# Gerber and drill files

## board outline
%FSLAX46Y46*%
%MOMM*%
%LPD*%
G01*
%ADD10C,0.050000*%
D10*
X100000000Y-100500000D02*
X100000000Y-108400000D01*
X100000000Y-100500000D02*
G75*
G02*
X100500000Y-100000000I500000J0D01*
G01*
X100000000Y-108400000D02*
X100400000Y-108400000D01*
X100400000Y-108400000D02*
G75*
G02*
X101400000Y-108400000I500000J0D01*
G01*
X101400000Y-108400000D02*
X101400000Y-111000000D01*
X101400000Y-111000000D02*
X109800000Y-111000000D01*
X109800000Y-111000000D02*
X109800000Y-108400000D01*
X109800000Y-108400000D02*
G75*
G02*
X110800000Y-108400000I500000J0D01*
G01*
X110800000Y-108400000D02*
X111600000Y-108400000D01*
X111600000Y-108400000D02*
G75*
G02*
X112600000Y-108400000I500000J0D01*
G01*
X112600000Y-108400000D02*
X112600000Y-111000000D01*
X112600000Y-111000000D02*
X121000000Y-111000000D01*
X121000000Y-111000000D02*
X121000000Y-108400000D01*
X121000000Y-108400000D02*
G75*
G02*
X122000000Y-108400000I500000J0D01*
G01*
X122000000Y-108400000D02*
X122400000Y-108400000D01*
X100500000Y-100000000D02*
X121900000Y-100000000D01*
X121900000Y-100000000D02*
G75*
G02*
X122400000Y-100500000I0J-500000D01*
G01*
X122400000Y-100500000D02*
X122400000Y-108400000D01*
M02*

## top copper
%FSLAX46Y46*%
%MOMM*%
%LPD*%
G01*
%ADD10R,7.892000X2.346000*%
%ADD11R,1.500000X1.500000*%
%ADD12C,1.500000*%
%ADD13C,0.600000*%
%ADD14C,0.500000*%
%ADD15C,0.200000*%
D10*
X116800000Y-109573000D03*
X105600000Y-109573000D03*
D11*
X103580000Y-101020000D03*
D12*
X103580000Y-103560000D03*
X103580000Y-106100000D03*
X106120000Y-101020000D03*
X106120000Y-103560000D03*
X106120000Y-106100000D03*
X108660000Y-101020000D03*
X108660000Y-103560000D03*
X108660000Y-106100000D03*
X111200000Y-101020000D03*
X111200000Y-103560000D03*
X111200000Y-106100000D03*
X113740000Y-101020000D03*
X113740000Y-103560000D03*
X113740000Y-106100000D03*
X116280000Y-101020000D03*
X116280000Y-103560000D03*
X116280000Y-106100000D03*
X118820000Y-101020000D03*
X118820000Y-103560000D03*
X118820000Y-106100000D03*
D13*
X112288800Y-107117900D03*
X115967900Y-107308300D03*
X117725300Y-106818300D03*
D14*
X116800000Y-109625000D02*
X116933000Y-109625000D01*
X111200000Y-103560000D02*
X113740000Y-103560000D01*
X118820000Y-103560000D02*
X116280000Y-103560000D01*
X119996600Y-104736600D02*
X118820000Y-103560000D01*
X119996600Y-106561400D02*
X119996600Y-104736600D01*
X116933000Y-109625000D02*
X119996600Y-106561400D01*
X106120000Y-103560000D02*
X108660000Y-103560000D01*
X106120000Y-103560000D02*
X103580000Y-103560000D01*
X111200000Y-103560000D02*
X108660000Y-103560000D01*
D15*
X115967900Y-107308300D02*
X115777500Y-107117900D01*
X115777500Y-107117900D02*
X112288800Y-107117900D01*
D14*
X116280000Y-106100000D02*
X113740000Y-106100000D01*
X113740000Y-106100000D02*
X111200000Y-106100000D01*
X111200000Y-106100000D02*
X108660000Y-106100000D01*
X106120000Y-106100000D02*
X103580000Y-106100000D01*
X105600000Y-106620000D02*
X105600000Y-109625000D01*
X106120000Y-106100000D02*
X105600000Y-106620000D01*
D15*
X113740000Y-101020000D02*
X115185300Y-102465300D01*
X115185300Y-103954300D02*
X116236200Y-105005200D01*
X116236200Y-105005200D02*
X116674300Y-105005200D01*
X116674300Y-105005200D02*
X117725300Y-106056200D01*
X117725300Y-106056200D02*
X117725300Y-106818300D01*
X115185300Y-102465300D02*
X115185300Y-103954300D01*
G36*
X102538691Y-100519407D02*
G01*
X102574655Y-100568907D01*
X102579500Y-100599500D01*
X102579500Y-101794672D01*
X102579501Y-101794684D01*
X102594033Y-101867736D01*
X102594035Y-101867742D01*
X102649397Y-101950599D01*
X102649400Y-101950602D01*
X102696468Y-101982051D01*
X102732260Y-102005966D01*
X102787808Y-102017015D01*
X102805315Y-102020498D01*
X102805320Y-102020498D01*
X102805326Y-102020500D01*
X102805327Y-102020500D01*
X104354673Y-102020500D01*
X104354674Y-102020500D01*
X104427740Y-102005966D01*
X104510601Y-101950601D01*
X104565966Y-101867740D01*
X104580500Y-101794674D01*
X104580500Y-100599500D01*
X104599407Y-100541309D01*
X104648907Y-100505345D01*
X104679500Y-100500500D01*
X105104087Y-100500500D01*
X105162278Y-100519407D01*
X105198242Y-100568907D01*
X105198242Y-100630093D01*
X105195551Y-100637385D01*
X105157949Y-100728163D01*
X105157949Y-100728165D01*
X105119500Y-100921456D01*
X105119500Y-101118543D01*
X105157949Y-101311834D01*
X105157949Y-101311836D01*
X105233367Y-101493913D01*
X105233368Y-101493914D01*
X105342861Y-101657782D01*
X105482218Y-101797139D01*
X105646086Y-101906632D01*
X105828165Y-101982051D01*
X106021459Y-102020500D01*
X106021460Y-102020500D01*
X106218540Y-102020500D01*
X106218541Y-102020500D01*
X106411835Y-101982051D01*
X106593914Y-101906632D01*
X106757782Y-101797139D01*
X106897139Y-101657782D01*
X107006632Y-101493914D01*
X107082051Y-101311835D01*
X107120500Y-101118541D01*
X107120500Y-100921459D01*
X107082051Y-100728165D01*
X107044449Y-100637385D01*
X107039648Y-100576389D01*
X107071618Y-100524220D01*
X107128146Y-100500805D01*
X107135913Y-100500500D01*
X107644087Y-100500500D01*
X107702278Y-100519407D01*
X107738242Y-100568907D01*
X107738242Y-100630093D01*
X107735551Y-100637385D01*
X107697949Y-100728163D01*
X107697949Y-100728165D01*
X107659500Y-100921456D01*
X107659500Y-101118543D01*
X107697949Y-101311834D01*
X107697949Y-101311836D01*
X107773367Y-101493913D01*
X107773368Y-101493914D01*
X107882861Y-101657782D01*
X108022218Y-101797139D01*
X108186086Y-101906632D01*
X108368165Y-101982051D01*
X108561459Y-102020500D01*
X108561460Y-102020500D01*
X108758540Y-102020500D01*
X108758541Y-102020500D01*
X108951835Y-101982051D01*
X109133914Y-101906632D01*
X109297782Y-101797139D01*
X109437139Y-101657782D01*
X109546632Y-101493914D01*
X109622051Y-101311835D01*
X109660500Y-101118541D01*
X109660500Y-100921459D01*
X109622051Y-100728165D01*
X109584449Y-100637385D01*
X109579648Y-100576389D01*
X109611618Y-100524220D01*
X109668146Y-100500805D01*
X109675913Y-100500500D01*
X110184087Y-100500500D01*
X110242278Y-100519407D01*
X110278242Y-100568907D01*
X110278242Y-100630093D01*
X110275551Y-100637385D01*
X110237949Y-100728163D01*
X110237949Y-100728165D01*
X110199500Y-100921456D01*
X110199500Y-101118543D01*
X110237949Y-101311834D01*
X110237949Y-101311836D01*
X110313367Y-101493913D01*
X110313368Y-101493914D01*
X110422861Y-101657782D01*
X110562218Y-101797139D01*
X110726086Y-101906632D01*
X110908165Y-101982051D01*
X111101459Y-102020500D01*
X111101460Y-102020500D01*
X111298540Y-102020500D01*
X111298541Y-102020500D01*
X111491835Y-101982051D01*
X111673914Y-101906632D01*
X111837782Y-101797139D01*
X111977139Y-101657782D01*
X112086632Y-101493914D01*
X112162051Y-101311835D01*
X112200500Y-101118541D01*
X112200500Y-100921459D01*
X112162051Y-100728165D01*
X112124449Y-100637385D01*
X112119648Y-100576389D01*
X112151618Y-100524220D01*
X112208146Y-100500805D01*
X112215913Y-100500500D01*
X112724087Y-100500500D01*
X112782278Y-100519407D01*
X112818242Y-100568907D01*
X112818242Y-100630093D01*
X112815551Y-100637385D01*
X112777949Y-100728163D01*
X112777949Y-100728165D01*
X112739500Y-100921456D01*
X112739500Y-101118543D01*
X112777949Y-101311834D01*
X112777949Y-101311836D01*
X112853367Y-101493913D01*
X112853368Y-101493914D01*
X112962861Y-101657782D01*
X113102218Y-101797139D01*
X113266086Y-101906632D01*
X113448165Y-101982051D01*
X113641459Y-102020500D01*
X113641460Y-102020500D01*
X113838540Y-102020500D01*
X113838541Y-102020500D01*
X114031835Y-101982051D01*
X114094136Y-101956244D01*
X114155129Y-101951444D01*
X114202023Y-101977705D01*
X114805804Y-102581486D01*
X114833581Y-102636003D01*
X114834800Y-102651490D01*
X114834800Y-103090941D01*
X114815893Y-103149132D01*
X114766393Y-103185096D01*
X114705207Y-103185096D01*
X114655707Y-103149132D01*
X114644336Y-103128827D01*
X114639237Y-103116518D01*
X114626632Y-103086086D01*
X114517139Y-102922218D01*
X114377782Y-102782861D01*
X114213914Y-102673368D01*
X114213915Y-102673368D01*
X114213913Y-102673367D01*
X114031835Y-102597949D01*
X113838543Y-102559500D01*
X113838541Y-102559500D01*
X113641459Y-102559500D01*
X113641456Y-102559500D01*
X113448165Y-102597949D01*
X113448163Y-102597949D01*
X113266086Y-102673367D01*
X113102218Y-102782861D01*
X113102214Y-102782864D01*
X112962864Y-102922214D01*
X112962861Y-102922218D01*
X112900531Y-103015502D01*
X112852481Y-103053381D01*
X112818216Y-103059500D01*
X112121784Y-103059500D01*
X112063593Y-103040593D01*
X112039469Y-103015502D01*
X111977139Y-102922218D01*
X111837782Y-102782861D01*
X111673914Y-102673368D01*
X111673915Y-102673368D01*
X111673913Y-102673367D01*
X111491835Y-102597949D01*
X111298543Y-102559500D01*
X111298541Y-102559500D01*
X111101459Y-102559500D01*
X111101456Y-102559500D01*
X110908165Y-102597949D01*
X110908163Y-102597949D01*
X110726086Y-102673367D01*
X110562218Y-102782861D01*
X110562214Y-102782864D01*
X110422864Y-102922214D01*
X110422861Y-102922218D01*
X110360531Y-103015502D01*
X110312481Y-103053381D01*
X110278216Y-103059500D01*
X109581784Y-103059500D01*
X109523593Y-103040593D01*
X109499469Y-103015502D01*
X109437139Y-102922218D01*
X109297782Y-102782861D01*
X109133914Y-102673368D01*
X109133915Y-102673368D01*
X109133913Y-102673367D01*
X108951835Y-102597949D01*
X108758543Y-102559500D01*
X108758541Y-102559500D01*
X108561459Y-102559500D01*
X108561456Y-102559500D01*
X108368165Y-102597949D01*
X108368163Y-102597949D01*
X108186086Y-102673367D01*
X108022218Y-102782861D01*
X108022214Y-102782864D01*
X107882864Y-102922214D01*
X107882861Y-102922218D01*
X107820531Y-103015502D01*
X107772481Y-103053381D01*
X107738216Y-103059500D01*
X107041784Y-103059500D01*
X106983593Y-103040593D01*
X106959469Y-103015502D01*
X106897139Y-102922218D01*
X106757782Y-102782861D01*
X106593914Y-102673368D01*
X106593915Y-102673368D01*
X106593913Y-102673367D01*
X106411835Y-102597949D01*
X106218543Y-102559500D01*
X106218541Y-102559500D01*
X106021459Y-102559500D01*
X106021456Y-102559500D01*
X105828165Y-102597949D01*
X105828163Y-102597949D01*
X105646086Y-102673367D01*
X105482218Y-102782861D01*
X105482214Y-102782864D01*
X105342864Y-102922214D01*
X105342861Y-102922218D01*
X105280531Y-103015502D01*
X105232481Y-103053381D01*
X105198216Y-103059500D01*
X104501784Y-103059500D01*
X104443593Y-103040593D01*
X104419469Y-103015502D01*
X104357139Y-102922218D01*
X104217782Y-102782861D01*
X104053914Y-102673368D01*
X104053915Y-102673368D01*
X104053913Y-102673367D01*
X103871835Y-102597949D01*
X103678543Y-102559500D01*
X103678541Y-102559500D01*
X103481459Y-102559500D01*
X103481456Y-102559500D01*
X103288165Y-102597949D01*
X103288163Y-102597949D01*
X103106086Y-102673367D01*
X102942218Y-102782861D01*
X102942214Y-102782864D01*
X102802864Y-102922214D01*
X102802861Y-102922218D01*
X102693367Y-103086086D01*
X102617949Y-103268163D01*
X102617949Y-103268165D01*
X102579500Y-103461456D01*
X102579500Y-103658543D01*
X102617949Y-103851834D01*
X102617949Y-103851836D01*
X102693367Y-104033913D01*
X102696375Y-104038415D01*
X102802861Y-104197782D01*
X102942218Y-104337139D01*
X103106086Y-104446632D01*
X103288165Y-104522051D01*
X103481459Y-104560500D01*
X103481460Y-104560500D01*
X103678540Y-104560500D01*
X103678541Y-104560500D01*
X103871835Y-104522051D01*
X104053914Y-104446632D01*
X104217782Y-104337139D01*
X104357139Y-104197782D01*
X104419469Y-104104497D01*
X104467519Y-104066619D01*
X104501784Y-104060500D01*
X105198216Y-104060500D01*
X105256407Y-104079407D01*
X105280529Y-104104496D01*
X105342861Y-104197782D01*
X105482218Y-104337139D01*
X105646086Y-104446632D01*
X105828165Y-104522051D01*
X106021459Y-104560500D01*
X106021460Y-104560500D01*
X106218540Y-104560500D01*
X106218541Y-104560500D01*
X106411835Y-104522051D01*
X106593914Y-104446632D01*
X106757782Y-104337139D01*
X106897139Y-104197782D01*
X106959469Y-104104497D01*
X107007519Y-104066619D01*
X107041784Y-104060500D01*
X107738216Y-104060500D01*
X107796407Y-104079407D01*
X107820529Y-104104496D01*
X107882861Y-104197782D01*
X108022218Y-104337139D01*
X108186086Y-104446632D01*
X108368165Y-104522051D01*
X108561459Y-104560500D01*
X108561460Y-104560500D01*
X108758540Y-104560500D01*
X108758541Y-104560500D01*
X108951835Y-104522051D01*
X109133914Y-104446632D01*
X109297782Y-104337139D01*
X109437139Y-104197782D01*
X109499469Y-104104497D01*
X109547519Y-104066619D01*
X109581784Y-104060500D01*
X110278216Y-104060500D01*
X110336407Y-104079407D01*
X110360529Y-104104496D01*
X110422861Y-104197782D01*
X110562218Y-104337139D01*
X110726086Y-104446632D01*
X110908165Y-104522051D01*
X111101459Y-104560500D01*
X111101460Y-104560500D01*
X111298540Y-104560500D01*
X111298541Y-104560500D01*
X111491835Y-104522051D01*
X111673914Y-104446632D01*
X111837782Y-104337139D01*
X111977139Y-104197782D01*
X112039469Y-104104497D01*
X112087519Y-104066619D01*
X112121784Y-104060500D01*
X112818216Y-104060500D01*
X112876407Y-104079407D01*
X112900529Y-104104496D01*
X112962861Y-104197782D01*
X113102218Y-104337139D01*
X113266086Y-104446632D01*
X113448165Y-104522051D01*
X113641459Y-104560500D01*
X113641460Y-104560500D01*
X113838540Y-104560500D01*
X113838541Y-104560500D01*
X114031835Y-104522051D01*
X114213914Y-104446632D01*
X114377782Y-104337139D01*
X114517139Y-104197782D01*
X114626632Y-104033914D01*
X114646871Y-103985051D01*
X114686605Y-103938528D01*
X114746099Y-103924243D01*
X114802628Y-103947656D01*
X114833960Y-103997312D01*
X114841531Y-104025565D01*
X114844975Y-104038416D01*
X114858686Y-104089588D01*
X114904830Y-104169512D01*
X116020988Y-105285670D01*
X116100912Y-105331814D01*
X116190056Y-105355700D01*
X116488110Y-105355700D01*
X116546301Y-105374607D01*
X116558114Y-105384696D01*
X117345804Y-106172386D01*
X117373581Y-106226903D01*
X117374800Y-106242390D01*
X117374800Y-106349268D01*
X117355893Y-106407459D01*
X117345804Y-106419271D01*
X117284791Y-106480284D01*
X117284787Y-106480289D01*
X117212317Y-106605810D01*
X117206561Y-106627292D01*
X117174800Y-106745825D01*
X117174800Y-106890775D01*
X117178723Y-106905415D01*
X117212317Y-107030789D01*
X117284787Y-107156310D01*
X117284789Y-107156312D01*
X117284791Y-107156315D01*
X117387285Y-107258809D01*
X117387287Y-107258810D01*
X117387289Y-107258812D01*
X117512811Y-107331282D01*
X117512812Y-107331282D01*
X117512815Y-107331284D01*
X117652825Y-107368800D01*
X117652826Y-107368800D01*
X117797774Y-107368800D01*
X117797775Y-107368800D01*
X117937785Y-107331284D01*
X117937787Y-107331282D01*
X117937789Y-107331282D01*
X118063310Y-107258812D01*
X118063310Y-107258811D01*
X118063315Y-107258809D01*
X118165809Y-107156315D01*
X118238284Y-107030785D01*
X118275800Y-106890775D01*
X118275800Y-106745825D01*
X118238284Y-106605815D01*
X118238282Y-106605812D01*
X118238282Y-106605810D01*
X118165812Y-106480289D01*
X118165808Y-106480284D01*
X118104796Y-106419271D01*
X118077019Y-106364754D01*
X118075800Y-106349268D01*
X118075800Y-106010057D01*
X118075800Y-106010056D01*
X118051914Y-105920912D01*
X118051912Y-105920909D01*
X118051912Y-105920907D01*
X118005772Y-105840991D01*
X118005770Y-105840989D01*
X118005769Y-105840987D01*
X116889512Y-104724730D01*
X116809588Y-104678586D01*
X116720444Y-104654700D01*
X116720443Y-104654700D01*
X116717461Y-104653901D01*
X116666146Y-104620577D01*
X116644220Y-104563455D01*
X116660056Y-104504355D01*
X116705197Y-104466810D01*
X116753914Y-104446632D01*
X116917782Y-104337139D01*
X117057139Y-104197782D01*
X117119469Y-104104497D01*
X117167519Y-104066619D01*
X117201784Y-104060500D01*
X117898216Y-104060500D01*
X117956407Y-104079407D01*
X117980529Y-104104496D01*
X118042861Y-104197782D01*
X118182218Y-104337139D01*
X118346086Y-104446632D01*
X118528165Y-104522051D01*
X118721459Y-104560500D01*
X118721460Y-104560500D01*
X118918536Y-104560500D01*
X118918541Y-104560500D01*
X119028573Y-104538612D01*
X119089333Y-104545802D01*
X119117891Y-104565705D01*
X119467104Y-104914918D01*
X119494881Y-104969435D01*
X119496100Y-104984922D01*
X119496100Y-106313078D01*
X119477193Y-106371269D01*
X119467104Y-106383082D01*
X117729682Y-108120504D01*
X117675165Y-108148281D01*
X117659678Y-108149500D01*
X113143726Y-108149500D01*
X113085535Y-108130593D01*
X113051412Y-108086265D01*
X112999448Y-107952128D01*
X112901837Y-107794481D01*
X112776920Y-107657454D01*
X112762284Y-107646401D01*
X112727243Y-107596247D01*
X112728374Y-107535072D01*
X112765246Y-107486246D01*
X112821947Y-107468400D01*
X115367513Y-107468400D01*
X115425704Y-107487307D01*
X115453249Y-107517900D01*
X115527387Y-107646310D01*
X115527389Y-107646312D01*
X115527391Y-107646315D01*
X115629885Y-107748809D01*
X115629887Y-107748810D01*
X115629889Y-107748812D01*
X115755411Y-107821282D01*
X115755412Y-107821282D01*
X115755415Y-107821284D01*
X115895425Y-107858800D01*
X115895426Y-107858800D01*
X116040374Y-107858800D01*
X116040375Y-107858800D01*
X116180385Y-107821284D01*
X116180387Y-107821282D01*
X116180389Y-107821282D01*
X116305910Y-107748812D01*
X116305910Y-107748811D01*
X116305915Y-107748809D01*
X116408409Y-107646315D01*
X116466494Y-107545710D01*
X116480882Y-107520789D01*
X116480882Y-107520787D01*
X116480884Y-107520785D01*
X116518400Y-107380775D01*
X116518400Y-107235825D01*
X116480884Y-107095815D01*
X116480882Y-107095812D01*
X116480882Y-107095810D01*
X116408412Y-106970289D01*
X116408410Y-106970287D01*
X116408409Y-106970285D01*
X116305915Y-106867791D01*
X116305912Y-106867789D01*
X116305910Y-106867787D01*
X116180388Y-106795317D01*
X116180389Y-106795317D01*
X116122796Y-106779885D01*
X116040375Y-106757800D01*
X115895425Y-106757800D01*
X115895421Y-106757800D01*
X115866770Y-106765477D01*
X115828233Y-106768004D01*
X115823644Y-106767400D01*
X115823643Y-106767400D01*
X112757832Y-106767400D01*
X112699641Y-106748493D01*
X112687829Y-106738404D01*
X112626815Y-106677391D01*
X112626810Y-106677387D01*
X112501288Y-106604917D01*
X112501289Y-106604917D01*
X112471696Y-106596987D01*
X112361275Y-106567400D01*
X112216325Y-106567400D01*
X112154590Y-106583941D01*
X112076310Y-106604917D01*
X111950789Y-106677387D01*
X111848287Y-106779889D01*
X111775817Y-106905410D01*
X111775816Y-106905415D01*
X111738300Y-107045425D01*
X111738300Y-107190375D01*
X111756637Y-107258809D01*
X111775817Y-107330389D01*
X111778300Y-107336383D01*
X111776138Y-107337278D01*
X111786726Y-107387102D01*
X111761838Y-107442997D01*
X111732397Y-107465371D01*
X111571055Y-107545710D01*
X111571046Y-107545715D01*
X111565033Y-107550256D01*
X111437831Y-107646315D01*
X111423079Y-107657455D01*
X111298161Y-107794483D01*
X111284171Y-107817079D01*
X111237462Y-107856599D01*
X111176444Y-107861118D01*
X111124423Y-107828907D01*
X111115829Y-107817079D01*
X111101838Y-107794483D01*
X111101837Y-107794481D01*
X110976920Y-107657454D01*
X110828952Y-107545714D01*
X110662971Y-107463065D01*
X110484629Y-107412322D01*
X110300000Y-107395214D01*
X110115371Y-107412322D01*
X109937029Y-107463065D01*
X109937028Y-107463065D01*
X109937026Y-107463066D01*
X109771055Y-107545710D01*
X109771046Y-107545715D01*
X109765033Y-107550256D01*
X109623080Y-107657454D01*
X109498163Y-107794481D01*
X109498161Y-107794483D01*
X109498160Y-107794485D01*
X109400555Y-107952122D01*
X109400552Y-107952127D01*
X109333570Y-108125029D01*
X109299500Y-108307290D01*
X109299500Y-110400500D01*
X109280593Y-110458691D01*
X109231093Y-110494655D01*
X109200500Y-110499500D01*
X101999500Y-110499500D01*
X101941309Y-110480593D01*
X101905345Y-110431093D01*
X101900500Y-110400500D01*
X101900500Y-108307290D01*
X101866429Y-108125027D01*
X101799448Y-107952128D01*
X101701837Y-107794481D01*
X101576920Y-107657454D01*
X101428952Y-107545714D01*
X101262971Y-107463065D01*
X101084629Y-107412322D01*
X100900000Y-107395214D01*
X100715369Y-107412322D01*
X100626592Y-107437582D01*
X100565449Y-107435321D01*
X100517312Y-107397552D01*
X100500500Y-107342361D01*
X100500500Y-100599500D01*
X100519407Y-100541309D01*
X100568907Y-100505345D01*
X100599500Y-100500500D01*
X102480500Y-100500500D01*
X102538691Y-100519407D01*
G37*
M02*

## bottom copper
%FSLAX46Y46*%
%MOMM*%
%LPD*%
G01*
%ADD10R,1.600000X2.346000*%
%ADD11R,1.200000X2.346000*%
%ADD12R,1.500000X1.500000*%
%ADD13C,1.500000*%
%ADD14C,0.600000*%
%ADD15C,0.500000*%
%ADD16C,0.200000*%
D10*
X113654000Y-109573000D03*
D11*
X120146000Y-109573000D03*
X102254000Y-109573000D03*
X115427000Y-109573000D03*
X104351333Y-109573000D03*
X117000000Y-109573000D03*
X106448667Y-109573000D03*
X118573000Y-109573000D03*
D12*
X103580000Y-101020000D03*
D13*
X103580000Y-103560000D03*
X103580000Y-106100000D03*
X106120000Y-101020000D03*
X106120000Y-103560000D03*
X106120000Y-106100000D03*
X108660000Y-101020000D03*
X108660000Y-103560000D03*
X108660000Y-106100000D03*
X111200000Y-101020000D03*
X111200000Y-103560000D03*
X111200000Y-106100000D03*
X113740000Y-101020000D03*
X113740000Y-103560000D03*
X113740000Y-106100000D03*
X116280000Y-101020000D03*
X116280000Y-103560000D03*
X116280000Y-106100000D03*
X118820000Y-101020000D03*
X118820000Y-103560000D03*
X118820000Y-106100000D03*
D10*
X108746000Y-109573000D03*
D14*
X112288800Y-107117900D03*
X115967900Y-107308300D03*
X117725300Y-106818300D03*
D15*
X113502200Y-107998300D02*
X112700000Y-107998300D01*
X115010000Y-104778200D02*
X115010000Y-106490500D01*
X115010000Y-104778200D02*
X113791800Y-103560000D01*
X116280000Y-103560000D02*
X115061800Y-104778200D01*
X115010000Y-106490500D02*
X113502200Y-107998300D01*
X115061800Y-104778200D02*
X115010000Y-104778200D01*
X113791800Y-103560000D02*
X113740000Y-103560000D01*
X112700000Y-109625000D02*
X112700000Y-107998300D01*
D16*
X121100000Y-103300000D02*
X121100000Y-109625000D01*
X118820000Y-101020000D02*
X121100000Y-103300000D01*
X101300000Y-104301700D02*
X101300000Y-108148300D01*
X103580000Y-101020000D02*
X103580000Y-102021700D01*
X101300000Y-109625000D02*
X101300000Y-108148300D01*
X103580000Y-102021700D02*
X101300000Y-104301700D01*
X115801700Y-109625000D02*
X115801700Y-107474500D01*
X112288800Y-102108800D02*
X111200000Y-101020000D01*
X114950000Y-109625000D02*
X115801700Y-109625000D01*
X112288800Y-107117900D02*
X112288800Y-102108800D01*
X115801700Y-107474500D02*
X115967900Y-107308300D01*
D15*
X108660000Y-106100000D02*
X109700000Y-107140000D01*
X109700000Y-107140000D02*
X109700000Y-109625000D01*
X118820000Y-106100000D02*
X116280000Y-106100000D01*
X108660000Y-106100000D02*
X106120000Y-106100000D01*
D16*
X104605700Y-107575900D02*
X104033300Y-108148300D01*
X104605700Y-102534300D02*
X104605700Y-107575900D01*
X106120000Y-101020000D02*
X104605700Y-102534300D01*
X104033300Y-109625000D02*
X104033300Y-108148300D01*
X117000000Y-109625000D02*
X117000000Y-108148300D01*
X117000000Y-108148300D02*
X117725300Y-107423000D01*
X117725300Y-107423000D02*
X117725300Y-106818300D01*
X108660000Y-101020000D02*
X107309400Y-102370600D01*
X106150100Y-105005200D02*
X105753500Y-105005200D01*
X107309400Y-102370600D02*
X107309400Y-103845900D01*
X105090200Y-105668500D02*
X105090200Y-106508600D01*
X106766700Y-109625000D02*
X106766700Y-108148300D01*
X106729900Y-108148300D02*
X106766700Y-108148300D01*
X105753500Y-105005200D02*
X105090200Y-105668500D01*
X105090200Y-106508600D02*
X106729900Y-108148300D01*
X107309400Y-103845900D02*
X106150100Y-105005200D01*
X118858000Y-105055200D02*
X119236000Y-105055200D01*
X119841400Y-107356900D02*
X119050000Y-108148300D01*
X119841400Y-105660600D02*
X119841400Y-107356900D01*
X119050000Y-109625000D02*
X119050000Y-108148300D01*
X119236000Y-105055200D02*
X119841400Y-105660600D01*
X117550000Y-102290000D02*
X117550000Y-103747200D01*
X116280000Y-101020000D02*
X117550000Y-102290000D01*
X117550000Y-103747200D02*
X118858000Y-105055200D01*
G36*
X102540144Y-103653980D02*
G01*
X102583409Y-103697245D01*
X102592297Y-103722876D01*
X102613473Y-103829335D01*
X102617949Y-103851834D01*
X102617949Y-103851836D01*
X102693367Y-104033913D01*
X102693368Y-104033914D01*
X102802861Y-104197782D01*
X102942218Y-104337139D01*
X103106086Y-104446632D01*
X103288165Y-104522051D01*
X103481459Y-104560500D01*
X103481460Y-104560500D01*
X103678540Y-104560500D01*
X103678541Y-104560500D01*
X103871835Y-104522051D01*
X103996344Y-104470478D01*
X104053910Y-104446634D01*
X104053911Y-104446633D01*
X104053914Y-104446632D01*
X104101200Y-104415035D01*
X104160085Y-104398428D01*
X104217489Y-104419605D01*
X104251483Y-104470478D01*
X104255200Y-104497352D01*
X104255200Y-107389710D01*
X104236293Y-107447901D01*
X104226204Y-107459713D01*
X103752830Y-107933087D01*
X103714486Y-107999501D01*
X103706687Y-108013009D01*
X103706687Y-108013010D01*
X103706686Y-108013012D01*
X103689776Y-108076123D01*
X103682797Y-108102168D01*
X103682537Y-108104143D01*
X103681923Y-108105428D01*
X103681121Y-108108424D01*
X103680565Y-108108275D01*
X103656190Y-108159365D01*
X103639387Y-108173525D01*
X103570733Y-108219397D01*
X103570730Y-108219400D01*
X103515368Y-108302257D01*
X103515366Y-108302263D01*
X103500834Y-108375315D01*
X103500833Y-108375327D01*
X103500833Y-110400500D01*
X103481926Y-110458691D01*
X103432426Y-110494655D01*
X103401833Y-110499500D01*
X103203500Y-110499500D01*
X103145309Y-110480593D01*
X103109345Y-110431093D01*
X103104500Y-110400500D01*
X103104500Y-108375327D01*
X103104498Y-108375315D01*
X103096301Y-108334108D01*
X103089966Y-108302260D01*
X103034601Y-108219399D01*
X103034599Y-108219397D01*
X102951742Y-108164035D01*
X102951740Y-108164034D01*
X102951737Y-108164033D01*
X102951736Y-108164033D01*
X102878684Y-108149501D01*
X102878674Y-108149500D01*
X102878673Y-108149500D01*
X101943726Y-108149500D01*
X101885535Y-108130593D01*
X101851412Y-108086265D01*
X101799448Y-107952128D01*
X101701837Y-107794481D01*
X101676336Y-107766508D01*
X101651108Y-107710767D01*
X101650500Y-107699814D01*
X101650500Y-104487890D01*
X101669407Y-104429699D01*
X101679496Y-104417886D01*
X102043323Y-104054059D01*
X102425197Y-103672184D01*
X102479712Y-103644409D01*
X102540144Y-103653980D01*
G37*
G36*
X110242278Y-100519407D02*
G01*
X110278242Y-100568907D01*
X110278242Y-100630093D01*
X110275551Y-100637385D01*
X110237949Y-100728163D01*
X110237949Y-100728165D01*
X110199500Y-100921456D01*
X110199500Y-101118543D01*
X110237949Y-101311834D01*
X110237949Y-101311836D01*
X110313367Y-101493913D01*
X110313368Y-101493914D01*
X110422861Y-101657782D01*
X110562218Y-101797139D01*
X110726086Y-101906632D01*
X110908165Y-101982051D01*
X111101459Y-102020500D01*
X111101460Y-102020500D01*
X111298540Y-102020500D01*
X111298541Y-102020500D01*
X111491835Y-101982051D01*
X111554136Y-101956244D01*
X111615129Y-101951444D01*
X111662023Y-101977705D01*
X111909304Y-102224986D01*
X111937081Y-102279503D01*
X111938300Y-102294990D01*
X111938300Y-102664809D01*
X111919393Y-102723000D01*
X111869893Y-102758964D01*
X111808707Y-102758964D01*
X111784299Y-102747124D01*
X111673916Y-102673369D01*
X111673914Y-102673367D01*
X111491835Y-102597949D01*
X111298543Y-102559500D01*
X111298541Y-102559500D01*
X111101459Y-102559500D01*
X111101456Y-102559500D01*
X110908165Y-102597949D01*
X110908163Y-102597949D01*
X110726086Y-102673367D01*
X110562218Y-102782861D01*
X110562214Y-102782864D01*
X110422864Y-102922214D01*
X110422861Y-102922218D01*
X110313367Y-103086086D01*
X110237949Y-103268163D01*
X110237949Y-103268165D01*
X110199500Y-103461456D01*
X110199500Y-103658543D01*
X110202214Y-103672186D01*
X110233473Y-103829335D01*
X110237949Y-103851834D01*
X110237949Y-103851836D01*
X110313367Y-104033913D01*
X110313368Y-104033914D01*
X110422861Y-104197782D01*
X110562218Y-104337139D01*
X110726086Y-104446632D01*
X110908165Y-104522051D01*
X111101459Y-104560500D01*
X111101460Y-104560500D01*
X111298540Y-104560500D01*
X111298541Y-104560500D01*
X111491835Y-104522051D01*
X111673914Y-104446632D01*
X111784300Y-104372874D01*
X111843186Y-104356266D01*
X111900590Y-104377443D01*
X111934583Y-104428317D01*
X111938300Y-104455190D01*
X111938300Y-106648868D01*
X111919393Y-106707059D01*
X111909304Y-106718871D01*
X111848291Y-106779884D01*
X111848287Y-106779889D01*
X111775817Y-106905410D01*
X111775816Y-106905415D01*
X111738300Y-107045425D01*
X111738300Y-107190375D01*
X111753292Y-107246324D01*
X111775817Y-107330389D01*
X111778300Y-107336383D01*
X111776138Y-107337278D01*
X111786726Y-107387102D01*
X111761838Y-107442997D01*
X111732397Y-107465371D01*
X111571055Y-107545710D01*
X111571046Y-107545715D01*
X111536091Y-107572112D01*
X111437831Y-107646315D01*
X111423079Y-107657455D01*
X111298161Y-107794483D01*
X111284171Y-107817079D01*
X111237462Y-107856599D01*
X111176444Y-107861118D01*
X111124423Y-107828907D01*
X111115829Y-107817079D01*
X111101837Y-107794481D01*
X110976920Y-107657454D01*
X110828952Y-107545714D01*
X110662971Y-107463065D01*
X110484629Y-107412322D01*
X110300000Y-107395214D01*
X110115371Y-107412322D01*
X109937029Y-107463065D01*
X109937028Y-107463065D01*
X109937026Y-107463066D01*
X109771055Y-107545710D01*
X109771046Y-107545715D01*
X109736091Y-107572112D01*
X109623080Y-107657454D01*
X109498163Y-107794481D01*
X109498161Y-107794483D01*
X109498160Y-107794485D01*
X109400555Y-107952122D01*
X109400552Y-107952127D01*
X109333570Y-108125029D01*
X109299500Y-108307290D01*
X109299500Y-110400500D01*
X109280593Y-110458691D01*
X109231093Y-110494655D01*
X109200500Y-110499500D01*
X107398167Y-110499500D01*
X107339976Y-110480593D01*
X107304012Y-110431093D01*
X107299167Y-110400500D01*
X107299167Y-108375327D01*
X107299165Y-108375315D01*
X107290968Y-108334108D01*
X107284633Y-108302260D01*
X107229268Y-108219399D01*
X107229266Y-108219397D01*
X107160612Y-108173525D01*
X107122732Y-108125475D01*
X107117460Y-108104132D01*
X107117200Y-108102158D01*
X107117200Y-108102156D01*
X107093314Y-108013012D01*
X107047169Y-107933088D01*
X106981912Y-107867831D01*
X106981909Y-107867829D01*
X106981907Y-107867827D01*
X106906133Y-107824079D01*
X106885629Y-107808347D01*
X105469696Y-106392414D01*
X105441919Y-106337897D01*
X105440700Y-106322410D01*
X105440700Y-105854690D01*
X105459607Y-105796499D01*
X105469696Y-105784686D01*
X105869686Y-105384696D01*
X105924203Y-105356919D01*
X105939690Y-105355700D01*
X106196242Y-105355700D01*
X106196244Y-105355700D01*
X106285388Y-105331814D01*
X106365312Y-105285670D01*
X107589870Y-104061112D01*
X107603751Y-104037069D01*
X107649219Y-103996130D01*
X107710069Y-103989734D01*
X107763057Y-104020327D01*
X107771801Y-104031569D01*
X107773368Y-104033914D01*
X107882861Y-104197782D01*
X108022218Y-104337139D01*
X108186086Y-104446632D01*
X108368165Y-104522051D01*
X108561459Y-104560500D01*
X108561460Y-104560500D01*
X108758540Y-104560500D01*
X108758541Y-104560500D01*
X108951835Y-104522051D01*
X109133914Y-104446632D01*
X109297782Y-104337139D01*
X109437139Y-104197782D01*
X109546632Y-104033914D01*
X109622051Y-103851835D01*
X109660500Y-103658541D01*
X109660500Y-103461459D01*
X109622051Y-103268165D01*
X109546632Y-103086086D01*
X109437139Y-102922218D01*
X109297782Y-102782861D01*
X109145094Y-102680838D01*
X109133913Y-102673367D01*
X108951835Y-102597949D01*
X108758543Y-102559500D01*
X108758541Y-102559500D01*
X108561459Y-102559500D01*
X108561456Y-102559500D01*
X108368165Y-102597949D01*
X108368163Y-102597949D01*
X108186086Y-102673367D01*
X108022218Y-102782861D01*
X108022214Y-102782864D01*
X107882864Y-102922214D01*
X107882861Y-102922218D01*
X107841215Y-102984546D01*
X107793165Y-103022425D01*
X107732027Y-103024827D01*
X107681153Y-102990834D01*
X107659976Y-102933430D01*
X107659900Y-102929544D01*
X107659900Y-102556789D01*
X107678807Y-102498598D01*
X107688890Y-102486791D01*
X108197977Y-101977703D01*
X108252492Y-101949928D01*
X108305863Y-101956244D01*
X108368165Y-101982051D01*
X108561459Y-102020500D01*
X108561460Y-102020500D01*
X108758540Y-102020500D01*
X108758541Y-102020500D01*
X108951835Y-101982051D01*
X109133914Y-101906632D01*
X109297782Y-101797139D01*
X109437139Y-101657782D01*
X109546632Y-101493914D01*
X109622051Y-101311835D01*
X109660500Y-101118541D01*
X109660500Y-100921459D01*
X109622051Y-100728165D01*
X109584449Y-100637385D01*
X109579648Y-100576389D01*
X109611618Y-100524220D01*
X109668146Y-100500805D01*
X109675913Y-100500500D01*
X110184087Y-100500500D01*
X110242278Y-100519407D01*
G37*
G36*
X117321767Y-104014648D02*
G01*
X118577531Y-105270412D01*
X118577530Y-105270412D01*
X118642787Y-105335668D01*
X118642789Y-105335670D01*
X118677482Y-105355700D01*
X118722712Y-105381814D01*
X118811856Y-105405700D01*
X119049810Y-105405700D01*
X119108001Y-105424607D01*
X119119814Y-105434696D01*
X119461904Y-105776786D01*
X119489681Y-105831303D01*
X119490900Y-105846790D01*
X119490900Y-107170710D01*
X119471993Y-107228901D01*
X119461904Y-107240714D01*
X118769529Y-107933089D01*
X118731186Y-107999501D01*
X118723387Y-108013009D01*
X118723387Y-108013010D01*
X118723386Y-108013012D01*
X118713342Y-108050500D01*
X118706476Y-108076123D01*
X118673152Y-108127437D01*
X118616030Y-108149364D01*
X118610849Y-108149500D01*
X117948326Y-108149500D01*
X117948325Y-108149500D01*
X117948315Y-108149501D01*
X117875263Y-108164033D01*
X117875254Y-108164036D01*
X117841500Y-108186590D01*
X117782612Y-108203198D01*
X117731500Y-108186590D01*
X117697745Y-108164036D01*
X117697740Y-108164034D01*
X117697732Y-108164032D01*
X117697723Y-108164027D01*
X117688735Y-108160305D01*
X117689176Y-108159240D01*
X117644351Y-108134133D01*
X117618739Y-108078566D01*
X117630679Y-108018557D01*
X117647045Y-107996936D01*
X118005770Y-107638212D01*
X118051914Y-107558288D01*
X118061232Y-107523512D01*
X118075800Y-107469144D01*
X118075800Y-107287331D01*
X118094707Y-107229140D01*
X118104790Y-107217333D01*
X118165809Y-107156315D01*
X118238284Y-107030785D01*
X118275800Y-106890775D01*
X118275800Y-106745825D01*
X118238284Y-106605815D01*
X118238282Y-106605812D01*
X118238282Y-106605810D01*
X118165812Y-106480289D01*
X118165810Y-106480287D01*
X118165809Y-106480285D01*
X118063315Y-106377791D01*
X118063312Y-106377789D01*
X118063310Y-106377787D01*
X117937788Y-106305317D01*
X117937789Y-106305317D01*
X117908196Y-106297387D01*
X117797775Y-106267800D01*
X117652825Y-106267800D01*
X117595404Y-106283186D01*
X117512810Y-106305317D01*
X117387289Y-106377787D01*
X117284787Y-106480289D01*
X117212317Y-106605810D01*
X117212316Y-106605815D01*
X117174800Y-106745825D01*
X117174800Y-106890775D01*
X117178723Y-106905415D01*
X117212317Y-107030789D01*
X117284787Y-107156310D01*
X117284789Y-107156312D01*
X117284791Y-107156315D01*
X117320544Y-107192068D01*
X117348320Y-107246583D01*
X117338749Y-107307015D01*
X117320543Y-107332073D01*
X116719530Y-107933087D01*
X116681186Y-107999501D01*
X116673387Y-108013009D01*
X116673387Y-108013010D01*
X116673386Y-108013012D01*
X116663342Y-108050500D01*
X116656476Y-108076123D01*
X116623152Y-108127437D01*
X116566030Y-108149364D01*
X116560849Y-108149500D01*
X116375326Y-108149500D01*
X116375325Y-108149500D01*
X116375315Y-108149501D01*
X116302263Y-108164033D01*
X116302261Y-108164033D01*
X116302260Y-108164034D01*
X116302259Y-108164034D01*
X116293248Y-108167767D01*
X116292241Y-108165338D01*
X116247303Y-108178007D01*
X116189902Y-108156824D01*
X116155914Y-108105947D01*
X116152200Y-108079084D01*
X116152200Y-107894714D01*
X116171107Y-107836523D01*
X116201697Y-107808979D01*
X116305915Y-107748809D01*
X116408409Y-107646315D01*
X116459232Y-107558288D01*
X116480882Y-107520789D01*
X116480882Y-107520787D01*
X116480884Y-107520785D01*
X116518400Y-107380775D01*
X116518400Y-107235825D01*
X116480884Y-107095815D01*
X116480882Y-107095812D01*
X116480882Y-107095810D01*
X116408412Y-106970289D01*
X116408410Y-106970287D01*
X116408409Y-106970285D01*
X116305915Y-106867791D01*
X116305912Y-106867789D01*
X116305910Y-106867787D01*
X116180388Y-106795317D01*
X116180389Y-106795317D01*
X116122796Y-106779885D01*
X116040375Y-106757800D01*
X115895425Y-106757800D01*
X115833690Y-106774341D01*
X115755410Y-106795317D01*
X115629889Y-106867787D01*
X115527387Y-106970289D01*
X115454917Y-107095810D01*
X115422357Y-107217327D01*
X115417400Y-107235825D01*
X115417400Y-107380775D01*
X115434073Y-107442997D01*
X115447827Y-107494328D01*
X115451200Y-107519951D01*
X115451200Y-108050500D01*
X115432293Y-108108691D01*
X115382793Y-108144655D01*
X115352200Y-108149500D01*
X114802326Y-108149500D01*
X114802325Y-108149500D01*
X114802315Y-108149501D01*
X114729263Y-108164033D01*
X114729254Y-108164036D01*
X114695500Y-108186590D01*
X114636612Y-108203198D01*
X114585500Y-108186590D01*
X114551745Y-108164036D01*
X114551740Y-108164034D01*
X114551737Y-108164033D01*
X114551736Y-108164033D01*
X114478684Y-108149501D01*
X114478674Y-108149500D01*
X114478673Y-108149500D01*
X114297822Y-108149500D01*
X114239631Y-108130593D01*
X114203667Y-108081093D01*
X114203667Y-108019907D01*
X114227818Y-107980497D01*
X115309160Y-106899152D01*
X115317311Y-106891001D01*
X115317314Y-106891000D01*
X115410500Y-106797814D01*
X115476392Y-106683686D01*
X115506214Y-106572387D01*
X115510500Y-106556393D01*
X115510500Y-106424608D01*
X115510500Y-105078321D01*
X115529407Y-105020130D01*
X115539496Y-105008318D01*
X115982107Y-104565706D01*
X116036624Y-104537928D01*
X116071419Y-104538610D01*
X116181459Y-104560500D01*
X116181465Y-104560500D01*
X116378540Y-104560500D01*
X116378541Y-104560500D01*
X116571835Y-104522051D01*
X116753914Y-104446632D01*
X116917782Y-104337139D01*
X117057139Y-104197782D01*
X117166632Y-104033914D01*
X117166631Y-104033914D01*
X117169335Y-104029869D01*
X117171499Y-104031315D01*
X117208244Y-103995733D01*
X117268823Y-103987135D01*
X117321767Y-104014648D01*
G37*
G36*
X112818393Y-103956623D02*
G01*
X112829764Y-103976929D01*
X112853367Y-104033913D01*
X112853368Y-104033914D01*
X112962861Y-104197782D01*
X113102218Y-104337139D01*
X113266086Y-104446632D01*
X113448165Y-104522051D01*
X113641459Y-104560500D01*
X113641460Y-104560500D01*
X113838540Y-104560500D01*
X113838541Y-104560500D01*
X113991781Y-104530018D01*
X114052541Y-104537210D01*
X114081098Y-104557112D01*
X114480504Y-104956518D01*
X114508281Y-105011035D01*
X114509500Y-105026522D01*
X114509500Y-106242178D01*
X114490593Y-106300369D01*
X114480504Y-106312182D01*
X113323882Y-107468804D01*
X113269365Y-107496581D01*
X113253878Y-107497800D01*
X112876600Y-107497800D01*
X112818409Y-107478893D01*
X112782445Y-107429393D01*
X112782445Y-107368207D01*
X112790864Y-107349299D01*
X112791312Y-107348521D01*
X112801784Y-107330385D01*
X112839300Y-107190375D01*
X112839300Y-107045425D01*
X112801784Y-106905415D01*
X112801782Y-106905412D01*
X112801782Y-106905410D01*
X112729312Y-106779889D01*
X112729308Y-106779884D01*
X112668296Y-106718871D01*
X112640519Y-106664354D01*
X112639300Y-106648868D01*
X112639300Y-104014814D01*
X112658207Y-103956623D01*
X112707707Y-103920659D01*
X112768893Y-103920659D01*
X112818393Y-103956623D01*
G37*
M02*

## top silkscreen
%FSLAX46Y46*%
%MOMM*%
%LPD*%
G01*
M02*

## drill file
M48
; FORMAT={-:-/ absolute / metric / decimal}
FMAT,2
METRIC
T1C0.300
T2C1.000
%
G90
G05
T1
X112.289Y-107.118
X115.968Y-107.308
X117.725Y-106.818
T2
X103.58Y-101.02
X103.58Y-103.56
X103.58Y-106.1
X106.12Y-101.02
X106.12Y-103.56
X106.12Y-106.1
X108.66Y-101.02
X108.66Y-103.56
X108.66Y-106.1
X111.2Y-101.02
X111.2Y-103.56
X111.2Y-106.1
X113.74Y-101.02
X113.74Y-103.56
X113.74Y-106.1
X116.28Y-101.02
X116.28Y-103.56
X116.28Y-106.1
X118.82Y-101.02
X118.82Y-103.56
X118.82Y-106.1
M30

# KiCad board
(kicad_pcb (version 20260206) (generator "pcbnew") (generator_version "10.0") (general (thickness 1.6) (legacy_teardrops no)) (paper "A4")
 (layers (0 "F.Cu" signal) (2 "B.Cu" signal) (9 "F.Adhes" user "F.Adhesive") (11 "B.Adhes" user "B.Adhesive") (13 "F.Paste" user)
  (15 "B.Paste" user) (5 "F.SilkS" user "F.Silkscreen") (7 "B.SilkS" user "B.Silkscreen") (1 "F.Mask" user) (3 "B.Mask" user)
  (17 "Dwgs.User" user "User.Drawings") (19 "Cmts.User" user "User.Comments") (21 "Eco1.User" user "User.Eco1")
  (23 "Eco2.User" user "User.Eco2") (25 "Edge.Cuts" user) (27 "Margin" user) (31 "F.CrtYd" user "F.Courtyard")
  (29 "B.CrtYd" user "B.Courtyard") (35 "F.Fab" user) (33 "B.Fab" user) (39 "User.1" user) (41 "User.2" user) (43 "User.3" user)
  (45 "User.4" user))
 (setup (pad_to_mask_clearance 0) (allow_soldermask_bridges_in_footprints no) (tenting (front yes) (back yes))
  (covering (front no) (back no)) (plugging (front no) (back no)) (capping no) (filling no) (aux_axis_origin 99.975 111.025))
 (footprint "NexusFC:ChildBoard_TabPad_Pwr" (layer "F.Cu") (at 113.654 108.4)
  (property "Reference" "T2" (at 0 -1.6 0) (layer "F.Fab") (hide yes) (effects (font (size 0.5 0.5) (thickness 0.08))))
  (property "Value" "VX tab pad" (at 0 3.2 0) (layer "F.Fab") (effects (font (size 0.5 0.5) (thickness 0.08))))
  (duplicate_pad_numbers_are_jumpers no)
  (pad "1" smd rect (at 0 1.173) (size 1.6 2.346) (layers "B.Cu" "B.Mask") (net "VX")))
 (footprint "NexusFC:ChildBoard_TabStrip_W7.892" (layer "F.Cu") (at 116.8 108.4)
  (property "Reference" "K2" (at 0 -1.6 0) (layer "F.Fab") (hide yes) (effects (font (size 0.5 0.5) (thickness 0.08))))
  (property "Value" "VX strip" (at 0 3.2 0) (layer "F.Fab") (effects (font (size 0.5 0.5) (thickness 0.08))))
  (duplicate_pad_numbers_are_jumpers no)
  (pad "1" smd rect (at 0 1.173) (size 7.892 2.346) (layers "F.Cu" "F.Mask") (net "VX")))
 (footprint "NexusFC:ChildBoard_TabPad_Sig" (layer "F.Cu") (at 120.146 108.4)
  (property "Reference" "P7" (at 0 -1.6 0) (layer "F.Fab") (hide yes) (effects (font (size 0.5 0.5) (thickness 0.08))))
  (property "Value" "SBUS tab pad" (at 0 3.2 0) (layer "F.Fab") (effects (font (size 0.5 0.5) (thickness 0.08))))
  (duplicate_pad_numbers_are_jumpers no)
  (pad "1" smd rect (at 0 1.173) (size 1.2 2.346) (layers "B.Cu" "B.Mask") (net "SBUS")))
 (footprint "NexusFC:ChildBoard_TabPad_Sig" (layer "F.Cu") (at 102.254 108.4)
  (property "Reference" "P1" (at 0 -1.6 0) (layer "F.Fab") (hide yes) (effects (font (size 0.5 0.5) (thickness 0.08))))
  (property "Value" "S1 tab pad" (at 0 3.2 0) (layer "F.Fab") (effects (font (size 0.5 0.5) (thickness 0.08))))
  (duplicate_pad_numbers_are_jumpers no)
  (pad "1" smd rect (at 0 1.173) (size 1.2 2.346) (layers "B.Cu" "B.Mask") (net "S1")))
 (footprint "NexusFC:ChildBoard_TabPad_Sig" (layer "F.Cu") (at 115.427 108.4)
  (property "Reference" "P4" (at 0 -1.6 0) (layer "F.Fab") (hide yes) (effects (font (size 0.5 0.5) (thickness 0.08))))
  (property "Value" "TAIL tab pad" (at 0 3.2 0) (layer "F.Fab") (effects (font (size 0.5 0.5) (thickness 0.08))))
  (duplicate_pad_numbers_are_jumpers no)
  (pad "1" smd rect (at 0 1.173) (size 1.2 2.346) (layers "B.Cu" "B.Mask") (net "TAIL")))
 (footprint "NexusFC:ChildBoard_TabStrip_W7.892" (layer "F.Cu") (at 105.6 108.4)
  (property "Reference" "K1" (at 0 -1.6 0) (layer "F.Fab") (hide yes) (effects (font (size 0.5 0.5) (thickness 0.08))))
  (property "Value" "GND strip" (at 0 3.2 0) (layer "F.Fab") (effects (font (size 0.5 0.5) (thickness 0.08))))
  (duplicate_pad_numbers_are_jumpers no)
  (pad "1" smd rect (at 0 1.173) (size 7.892 2.346) (layers "F.Cu" "F.Mask") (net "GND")))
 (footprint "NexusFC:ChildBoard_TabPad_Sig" (layer "F.Cu") (at 104.351333 108.4)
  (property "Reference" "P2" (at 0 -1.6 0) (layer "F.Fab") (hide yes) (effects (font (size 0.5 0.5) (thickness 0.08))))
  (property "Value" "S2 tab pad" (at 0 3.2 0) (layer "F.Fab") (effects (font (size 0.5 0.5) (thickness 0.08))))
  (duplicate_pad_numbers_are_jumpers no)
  (pad "1" smd rect (at 0 1.173) (size 1.2 2.346) (layers "B.Cu" "B.Mask") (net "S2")))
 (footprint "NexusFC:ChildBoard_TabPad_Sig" (layer "F.Cu") (at 117 108.4)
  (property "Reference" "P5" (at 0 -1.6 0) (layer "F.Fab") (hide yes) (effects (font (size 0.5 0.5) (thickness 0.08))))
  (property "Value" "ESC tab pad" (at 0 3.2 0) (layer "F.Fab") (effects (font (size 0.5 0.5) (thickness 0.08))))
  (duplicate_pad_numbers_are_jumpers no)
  (pad "1" smd rect (at 0 1.173) (size 1.2 2.346) (layers "B.Cu" "B.Mask") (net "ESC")))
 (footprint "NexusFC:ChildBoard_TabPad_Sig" (layer "F.Cu") (at 106.448667 108.4)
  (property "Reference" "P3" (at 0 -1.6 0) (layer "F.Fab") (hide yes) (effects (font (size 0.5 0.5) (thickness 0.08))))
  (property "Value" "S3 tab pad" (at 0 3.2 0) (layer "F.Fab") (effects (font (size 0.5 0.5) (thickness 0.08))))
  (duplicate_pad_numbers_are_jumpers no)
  (pad "1" smd rect (at 0 1.173) (size 1.2 2.346) (layers "B.Cu" "B.Mask") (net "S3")))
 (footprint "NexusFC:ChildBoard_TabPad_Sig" (layer "F.Cu") (at 118.573 108.4)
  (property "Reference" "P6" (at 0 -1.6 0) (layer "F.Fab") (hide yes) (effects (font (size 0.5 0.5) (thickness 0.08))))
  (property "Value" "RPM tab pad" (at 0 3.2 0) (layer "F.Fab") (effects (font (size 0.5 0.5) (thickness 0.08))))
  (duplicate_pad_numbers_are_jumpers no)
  (pad "1" smd rect (at 0 1.173) (size 1.2 2.346) (layers "B.Cu" "B.Mask") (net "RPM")))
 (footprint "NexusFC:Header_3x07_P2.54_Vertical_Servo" (layer "F.Cu") (at 111.2 103.56)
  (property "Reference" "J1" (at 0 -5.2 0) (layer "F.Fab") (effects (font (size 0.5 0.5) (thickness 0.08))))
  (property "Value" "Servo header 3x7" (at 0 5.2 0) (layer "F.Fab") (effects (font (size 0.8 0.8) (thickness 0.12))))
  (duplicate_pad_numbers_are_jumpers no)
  (pad "1" thru_hole rect (at -7.62 -2.54) (size 1.5 1.5) (drill 1) (layers "*.Cu" "*.Mask") (remove_unused_layers no) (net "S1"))
  (pad "2" thru_hole circle (at -7.62 0) (size 1.5 1.5) (drill 1) (layers "*.Cu" "*.Mask") (remove_unused_layers no) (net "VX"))
  (pad "3" thru_hole circle (at -7.62 2.54) (size 1.5 1.5) (drill 1) (layers "*.Cu" "*.Mask") (remove_unused_layers no) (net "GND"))
  (pad "4" thru_hole circle (at -5.08 -2.54) (size 1.5 1.5) (drill 1) (layers "*.Cu" "*.Mask") (remove_unused_layers no) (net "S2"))
  (pad "5" thru_hole circle (at -5.08 0) (size 1.5 1.5) (drill 1) (layers "*.Cu" "*.Mask") (remove_unused_layers no) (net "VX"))
  (pad "6" thru_hole circle (at -5.08 2.54) (size 1.5 1.5) (drill 1) (layers "*.Cu" "*.Mask") (remove_unused_layers no) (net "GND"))
  (pad "7" thru_hole circle (at -2.54 -2.54) (size 1.5 1.5) (drill 1) (layers "*.Cu" "*.Mask") (remove_unused_layers no) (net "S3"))
  (pad "8" thru_hole circle (at -2.54 0) (size 1.5 1.5) (drill 1) (layers "*.Cu" "*.Mask") (remove_unused_layers no) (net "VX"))
  (pad "9" thru_hole circle (at -2.54 2.54) (size 1.5 1.5) (drill 1) (layers "*.Cu" "*.Mask") (remove_unused_layers no) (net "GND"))
  (pad "10" thru_hole circle (at 0 -2.54) (size 1.5 1.5) (drill 1) (layers "*.Cu" "*.Mask") (remove_unused_layers no) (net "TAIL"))
  (pad "11" thru_hole circle (at 0 0) (size 1.5 1.5) (drill 1) (layers "*.Cu" "*.Mask") (remove_unused_layers no) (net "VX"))
  (pad "12" thru_hole circle (at 0 2.54) (size 1.5 1.5) (drill 1) (layers "*.Cu" "*.Mask") (remove_unused_layers no) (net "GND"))
  (pad "13" thru_hole circle (at 2.54 -2.54) (size 1.5 1.5) (drill 1) (layers "*.Cu" "*.Mask") (remove_unused_layers no) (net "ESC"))
  (pad "14" thru_hole circle (at 2.54 0) (size 1.5 1.5) (drill 1) (layers "*.Cu" "*.Mask") (remove_unused_layers no) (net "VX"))
  (pad "15" thru_hole circle (at 2.54 2.54) (size 1.5 1.5) (drill 1) (layers "*.Cu" "*.Mask") (remove_unused_layers no) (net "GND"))
  (pad "16" thru_hole circle (at 5.08 -2.54) (size 1.5 1.5) (drill 1) (layers "*.Cu" "*.Mask") (remove_unused_layers no) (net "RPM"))
  (pad "17" thru_hole circle (at 5.08 0) (size 1.5 1.5) (drill 1) (layers "*.Cu" "*.Mask") (remove_unused_layers no) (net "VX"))
  (pad "18" thru_hole circle (at 5.08 2.54) (size 1.5 1.5) (drill 1) (layers "*.Cu" "*.Mask") (remove_unused_layers no) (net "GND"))
  (pad "19" thru_hole circle (at 7.62 -2.54) (size 1.5 1.5) (drill 1) (layers "*.Cu" "*.Mask") (remove_unused_layers no) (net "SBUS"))
  (pad "20" thru_hole circle (at 7.62 0) (size 1.5 1.5) (drill 1) (layers "*.Cu" "*.Mask") (remove_unused_layers no) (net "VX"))
  (pad "21" thru_hole circle (at 7.62 2.54) (size 1.5 1.5) (drill 1) (layers "*.Cu" "*.Mask") (remove_unused_layers no) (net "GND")))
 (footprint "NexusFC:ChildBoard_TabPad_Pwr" (layer "F.Cu") (at 108.746 108.4)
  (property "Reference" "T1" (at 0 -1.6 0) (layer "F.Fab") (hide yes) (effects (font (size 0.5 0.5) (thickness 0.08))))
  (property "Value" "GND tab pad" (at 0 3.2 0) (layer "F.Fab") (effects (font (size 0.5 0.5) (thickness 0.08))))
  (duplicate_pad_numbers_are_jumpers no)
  (pad "1" smd rect (at 0 1.173) (size 1.6 2.346) (layers "B.Cu" "B.Mask") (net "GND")))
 (gr_line (start 100 100.5) (end 100 108.4) (stroke (width 0.05) (type default)) (layer "Edge.Cuts"))
 (gr_arc (start 100 100.5) (mid 100.146447 100.146447) (end 100.5 100) (stroke (width 0.05) (type default)) (layer "Edge.Cuts"))
 (gr_line (start 100.000000 108.400000) (end 100.400000 108.400000) (stroke (width 0.05) (type solid)) (layer "Edge.Cuts"))
 (gr_arc (start 100.400000 108.400000) (mid 100.900000 107.900000) (end 101.400000 108.400000) (stroke (width 0.05) (type solid))
  (layer "Edge.Cuts"))
 (gr_line (start 101.400000 108.400000) (end 101.400000 111.000000) (stroke (width 0.05) (type solid)) (layer "Edge.Cuts"))
 (gr_line (start 101.400000 111.000000) (end 109.800000 111.000000) (stroke (width 0.05) (type solid)) (layer "Edge.Cuts"))
 (gr_line (start 109.800000 111.000000) (end 109.800000 108.400000) (stroke (width 0.05) (type solid)) (layer "Edge.Cuts"))
 (gr_arc (start 109.800000 108.400000) (mid 110.300000 107.900000) (end 110.800000 108.400000) (stroke (width 0.05) (type solid))
  (layer "Edge.Cuts"))
 (gr_line (start 110.800000 108.400000) (end 111.600000 108.400000) (stroke (width 0.05) (type solid)) (layer "Edge.Cuts"))
 (gr_arc (start 111.600000 108.400000) (mid 112.100000 107.900000) (end 112.600000 108.400000) (stroke (width 0.05) (type solid))
  (layer "Edge.Cuts"))
 (gr_line (start 112.600000 108.400000) (end 112.600000 111.000000) (stroke (width 0.05) (type solid)) (layer "Edge.Cuts"))
 (gr_line (start 112.600000 111.000000) (end 121.000000 111.000000) (stroke (width 0.05) (type solid)) (layer "Edge.Cuts"))
 (gr_line (start 121.000000 111.000000) (end 121.000000 108.400000) (stroke (width 0.05) (type solid)) (layer "Edge.Cuts"))
 (gr_arc (start 121.000000 108.400000) (mid 121.500000 107.900000) (end 122.000000 108.400000) (stroke (width 0.05) (type solid))
  (layer "Edge.Cuts"))
 (gr_line (start 122.000000 108.400000) (end 122.400000 108.400000) (stroke (width 0.05) (type solid)) (layer "Edge.Cuts"))
 (gr_line (start 100.5 100) (end 121.9 100) (stroke (width 0.05) (type default)) (layer "Edge.Cuts"))
 (gr_arc (start 121.9 100) (mid 122.253553 100.146447) (end 122.4 100.5) (stroke (width 0.05) (type default)) (layer "Edge.Cuts"))
 (gr_line (start 122.4 100.5) (end 122.4 108.4) (stroke (width 0.05) (type default)) (layer "Edge.Cuts"))
 (segment (start 116.8 109.625) (end 116.933 109.625) (width 0.5) (layer "F.Cu") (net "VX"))
 (segment (start 111.2 103.56) (end 113.74 103.56) (width 0.5) (layer "F.Cu") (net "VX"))
 (segment (start 118.82 103.56) (end 116.28 103.56) (width 0.5) (layer "F.Cu") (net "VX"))
 (segment (start 119.9966 104.7366) (end 118.82 103.56) (width 0.5) (layer "F.Cu") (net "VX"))
 (segment (start 119.9966 106.5614) (end 119.9966 104.7366) (width 0.5) (layer "F.Cu") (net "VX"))
 (segment (start 116.933 109.625) (end 119.9966 106.5614) (width 0.5) (layer "F.Cu") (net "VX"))
 (segment (start 106.12 103.56) (end 108.66 103.56) (width 0.5) (layer "F.Cu") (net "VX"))
 (segment (start 106.12 103.56) (end 103.58 103.56) (width 0.5) (layer "F.Cu") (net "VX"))
 (segment (start 111.2 103.56) (end 108.66 103.56) (width 0.5) (layer "F.Cu") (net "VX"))
 (segment (start 113.5022 107.9983) (end 112.7 107.9983) (width 0.5) (layer "B.Cu") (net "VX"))
 (segment (start 115.01 104.7782) (end 115.01 106.4905) (width 0.5) (layer "B.Cu") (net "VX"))
 (segment (start 115.01 104.7782) (end 113.7918 103.56) (width 0.5) (layer "B.Cu") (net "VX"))
 (segment (start 116.28 103.56) (end 115.0618 104.7782) (width 0.5) (layer "B.Cu") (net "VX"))
 (segment (start 115.01 106.4905) (end 113.5022 107.9983) (width 0.5) (layer "B.Cu") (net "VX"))
 (segment (start 115.0618 104.7782) (end 115.01 104.7782) (width 0.5) (layer "B.Cu") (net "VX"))
 (segment (start 113.7918 103.56) (end 113.74 103.56) (width 0.5) (layer "B.Cu") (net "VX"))
 (segment (start 112.7 109.625) (end 112.7 107.9983) (width 0.5) (layer "B.Cu") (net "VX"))
 (segment (start 121.1 103.3) (end 121.1 109.625) (width 0.2) (layer "B.Cu") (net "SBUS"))
 (segment (start 118.82 101.02) (end 121.1 103.3) (width 0.2) (layer "B.Cu") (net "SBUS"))
 (segment (start 101.3 104.3017) (end 101.3 108.1483) (width 0.2) (layer "B.Cu") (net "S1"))
 (segment (start 103.58 101.02) (end 103.58 102.0217) (width 0.2) (layer "B.Cu") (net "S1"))
 (segment (start 101.3 109.625) (end 101.3 108.1483) (width 0.2) (layer "B.Cu") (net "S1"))
 (segment (start 103.58 102.0217) (end 101.3 104.3017) (width 0.2) (layer "B.Cu") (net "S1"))
 (segment (start 115.9679 107.3083) (end 115.7775 107.1179) (width 0.2) (layer "F.Cu") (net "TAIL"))
 (segment (start 115.7775 107.1179) (end 112.2888 107.1179) (width 0.2) (layer "F.Cu") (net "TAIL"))
 (via (at 112.2888 107.1179) (size 0.6) (drill 0.3) (layers "F.Cu" "B.Cu") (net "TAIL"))
 (via (at 115.9679 107.3083) (size 0.6) (drill 0.3) (layers "F.Cu" "B.Cu") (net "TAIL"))
 (segment (start 115.8017 109.625) (end 115.8017 107.4745) (width 0.2) (layer "B.Cu") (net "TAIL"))
 (segment (start 112.2888 102.1088) (end 111.2 101.02) (width 0.2) (layer "B.Cu") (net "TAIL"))
 (segment (start 114.95 109.625) (end 115.8017 109.625) (width 0.2) (layer "B.Cu") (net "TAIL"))
 (segment (start 112.2888 107.1179) (end 112.2888 102.1088) (width 0.2) (layer "B.Cu") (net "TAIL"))
 (segment (start 115.8017 107.4745) (end 115.9679 107.3083) (width 0.2) (layer "B.Cu") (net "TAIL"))
 (segment (start 116.28 106.1) (end 113.74 106.1) (width 0.5) (layer "F.Cu") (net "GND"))
 (segment (start 113.74 106.1) (end 111.2 106.1) (width 0.5) (layer "F.Cu") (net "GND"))
 (segment (start 111.2 106.1) (end 108.66 106.1) (width 0.5) (layer "F.Cu") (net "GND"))
 (segment (start 106.12 106.1) (end 103.58 106.1) (width 0.5) (layer "F.Cu") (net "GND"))
 (segment (start 105.6 106.62) (end 105.6 109.625) (width 0.5) (layer "F.Cu") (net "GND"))
 (segment (start 106.12 106.1) (end 105.6 106.62) (width 0.5) (layer "F.Cu") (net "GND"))
 (segment (start 108.66 106.1) (end 109.7 107.14) (width 0.5) (layer "B.Cu") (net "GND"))
 (segment (start 109.7 107.14) (end 109.7 109.625) (width 0.5) (layer "B.Cu") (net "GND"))
 (segment (start 118.82 106.1) (end 116.28 106.1) (width 0.5) (layer "B.Cu") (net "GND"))
 (segment (start 108.66 106.1) (end 106.12 106.1) (width 0.5) (layer "B.Cu") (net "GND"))
 (segment (start 104.6057 107.5759) (end 104.0333 108.1483) (width 0.2) (layer "B.Cu") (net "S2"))
 (segment (start 104.6057 102.5343) (end 104.6057 107.5759) (width 0.2) (layer "B.Cu") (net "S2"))
 (segment (start 106.12 101.02) (end 104.6057 102.5343) (width 0.2) (layer "B.Cu") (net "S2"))
 (segment (start 104.0333 109.625) (end 104.0333 108.1483) (width 0.2) (layer "B.Cu") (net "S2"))
 (segment (start 113.74 101.02) (end 115.1853 102.4653) (width 0.2) (layer "F.Cu") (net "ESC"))
 (segment (start 115.1853 103.9543) (end 116.2362 105.0052) (width 0.2) (layer "F.Cu") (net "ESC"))
 (segment (start 116.2362 105.0052) (end 116.6743 105.0052) (width 0.2) (layer "F.Cu") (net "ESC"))
 (segment (start 116.6743 105.0052) (end 117.7253 106.0562) (width 0.2) (layer "F.Cu") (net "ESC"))
 (segment (start 117.7253 106.0562) (end 117.7253 106.8183) (width 0.2) (layer "F.Cu") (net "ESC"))
 (segment (start 115.1853 102.4653) (end 115.1853 103.9543) (width 0.2) (layer "F.Cu") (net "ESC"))
 (via (at 117.7253 106.8183) (size 0.6) (drill 0.3) (layers "F.Cu" "B.Cu") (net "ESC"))
 (segment (start 117 109.625) (end 117 108.1483) (width 0.2) (layer "B.Cu") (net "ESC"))
 (segment (start 117 108.1483) (end 117.7253 107.423) (width 0.2) (layer "B.Cu") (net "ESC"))
 (segment (start 117.7253 107.423) (end 117.7253 106.8183) (width 0.2) (layer "B.Cu") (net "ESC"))
 (segment (start 108.66 101.02) (end 107.3094 102.3706) (width 0.2) (layer "B.Cu") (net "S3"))
 (segment (start 106.1501 105.0052) (end 105.7535 105.0052) (width 0.2) (layer "B.Cu") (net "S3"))
 (segment (start 107.3094 102.3706) (end 107.3094 103.8459) (width 0.2) (layer "B.Cu") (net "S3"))
 (segment (start 105.0902 105.6685) (end 105.0902 106.5086) (width 0.2) (layer "B.Cu") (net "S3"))
 (segment (start 106.7667 109.625) (end 106.7667 108.1483) (width 0.2) (layer "B.Cu") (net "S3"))
 (segment (start 106.7299 108.1483) (end 106.7667 108.1483) (width 0.2) (layer "B.Cu") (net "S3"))
 (segment (start 105.7535 105.0052) (end 105.0902 105.6685) (width 0.2) (layer "B.Cu") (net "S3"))
 (segment (start 105.0902 106.5086) (end 106.7299 108.1483) (width 0.2) (layer "B.Cu") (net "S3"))
 (segment (start 107.3094 103.8459) (end 106.1501 105.0052) (width 0.2) (layer "B.Cu") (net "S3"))
 (segment (start 118.858 105.0552) (end 119.236 105.0552) (width 0.2) (layer "B.Cu") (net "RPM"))
 (segment (start 119.8414 107.3569) (end 119.05 108.1483) (width 0.2) (layer "B.Cu") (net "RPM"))
 (segment (start 119.8414 105.6606) (end 119.8414 107.3569) (width 0.2) (layer "B.Cu") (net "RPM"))
 (segment (start 119.05 109.625) (end 119.05 108.1483) (width 0.2) (layer "B.Cu") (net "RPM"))
 (segment (start 119.236 105.0552) (end 119.8414 105.6606) (width 0.2) (layer "B.Cu") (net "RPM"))
 (segment (start 117.55 102.29) (end 117.55 103.7472) (width 0.2) (layer "B.Cu") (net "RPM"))
 (segment (start 116.28 101.02) (end 117.55 102.29) (width 0.2) (layer "B.Cu") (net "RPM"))
 (segment (start 117.55 103.7472) (end 118.858 105.0552) (width 0.2) (layer "B.Cu") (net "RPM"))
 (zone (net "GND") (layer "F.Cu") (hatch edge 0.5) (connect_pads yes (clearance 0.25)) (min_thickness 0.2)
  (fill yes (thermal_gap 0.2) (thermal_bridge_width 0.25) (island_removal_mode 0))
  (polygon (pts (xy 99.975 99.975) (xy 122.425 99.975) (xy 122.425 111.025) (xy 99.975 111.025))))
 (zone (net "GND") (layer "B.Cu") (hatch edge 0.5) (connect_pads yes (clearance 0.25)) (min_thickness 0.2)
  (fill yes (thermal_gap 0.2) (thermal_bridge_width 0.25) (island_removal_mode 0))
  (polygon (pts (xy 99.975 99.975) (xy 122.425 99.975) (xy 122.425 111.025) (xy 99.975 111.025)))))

